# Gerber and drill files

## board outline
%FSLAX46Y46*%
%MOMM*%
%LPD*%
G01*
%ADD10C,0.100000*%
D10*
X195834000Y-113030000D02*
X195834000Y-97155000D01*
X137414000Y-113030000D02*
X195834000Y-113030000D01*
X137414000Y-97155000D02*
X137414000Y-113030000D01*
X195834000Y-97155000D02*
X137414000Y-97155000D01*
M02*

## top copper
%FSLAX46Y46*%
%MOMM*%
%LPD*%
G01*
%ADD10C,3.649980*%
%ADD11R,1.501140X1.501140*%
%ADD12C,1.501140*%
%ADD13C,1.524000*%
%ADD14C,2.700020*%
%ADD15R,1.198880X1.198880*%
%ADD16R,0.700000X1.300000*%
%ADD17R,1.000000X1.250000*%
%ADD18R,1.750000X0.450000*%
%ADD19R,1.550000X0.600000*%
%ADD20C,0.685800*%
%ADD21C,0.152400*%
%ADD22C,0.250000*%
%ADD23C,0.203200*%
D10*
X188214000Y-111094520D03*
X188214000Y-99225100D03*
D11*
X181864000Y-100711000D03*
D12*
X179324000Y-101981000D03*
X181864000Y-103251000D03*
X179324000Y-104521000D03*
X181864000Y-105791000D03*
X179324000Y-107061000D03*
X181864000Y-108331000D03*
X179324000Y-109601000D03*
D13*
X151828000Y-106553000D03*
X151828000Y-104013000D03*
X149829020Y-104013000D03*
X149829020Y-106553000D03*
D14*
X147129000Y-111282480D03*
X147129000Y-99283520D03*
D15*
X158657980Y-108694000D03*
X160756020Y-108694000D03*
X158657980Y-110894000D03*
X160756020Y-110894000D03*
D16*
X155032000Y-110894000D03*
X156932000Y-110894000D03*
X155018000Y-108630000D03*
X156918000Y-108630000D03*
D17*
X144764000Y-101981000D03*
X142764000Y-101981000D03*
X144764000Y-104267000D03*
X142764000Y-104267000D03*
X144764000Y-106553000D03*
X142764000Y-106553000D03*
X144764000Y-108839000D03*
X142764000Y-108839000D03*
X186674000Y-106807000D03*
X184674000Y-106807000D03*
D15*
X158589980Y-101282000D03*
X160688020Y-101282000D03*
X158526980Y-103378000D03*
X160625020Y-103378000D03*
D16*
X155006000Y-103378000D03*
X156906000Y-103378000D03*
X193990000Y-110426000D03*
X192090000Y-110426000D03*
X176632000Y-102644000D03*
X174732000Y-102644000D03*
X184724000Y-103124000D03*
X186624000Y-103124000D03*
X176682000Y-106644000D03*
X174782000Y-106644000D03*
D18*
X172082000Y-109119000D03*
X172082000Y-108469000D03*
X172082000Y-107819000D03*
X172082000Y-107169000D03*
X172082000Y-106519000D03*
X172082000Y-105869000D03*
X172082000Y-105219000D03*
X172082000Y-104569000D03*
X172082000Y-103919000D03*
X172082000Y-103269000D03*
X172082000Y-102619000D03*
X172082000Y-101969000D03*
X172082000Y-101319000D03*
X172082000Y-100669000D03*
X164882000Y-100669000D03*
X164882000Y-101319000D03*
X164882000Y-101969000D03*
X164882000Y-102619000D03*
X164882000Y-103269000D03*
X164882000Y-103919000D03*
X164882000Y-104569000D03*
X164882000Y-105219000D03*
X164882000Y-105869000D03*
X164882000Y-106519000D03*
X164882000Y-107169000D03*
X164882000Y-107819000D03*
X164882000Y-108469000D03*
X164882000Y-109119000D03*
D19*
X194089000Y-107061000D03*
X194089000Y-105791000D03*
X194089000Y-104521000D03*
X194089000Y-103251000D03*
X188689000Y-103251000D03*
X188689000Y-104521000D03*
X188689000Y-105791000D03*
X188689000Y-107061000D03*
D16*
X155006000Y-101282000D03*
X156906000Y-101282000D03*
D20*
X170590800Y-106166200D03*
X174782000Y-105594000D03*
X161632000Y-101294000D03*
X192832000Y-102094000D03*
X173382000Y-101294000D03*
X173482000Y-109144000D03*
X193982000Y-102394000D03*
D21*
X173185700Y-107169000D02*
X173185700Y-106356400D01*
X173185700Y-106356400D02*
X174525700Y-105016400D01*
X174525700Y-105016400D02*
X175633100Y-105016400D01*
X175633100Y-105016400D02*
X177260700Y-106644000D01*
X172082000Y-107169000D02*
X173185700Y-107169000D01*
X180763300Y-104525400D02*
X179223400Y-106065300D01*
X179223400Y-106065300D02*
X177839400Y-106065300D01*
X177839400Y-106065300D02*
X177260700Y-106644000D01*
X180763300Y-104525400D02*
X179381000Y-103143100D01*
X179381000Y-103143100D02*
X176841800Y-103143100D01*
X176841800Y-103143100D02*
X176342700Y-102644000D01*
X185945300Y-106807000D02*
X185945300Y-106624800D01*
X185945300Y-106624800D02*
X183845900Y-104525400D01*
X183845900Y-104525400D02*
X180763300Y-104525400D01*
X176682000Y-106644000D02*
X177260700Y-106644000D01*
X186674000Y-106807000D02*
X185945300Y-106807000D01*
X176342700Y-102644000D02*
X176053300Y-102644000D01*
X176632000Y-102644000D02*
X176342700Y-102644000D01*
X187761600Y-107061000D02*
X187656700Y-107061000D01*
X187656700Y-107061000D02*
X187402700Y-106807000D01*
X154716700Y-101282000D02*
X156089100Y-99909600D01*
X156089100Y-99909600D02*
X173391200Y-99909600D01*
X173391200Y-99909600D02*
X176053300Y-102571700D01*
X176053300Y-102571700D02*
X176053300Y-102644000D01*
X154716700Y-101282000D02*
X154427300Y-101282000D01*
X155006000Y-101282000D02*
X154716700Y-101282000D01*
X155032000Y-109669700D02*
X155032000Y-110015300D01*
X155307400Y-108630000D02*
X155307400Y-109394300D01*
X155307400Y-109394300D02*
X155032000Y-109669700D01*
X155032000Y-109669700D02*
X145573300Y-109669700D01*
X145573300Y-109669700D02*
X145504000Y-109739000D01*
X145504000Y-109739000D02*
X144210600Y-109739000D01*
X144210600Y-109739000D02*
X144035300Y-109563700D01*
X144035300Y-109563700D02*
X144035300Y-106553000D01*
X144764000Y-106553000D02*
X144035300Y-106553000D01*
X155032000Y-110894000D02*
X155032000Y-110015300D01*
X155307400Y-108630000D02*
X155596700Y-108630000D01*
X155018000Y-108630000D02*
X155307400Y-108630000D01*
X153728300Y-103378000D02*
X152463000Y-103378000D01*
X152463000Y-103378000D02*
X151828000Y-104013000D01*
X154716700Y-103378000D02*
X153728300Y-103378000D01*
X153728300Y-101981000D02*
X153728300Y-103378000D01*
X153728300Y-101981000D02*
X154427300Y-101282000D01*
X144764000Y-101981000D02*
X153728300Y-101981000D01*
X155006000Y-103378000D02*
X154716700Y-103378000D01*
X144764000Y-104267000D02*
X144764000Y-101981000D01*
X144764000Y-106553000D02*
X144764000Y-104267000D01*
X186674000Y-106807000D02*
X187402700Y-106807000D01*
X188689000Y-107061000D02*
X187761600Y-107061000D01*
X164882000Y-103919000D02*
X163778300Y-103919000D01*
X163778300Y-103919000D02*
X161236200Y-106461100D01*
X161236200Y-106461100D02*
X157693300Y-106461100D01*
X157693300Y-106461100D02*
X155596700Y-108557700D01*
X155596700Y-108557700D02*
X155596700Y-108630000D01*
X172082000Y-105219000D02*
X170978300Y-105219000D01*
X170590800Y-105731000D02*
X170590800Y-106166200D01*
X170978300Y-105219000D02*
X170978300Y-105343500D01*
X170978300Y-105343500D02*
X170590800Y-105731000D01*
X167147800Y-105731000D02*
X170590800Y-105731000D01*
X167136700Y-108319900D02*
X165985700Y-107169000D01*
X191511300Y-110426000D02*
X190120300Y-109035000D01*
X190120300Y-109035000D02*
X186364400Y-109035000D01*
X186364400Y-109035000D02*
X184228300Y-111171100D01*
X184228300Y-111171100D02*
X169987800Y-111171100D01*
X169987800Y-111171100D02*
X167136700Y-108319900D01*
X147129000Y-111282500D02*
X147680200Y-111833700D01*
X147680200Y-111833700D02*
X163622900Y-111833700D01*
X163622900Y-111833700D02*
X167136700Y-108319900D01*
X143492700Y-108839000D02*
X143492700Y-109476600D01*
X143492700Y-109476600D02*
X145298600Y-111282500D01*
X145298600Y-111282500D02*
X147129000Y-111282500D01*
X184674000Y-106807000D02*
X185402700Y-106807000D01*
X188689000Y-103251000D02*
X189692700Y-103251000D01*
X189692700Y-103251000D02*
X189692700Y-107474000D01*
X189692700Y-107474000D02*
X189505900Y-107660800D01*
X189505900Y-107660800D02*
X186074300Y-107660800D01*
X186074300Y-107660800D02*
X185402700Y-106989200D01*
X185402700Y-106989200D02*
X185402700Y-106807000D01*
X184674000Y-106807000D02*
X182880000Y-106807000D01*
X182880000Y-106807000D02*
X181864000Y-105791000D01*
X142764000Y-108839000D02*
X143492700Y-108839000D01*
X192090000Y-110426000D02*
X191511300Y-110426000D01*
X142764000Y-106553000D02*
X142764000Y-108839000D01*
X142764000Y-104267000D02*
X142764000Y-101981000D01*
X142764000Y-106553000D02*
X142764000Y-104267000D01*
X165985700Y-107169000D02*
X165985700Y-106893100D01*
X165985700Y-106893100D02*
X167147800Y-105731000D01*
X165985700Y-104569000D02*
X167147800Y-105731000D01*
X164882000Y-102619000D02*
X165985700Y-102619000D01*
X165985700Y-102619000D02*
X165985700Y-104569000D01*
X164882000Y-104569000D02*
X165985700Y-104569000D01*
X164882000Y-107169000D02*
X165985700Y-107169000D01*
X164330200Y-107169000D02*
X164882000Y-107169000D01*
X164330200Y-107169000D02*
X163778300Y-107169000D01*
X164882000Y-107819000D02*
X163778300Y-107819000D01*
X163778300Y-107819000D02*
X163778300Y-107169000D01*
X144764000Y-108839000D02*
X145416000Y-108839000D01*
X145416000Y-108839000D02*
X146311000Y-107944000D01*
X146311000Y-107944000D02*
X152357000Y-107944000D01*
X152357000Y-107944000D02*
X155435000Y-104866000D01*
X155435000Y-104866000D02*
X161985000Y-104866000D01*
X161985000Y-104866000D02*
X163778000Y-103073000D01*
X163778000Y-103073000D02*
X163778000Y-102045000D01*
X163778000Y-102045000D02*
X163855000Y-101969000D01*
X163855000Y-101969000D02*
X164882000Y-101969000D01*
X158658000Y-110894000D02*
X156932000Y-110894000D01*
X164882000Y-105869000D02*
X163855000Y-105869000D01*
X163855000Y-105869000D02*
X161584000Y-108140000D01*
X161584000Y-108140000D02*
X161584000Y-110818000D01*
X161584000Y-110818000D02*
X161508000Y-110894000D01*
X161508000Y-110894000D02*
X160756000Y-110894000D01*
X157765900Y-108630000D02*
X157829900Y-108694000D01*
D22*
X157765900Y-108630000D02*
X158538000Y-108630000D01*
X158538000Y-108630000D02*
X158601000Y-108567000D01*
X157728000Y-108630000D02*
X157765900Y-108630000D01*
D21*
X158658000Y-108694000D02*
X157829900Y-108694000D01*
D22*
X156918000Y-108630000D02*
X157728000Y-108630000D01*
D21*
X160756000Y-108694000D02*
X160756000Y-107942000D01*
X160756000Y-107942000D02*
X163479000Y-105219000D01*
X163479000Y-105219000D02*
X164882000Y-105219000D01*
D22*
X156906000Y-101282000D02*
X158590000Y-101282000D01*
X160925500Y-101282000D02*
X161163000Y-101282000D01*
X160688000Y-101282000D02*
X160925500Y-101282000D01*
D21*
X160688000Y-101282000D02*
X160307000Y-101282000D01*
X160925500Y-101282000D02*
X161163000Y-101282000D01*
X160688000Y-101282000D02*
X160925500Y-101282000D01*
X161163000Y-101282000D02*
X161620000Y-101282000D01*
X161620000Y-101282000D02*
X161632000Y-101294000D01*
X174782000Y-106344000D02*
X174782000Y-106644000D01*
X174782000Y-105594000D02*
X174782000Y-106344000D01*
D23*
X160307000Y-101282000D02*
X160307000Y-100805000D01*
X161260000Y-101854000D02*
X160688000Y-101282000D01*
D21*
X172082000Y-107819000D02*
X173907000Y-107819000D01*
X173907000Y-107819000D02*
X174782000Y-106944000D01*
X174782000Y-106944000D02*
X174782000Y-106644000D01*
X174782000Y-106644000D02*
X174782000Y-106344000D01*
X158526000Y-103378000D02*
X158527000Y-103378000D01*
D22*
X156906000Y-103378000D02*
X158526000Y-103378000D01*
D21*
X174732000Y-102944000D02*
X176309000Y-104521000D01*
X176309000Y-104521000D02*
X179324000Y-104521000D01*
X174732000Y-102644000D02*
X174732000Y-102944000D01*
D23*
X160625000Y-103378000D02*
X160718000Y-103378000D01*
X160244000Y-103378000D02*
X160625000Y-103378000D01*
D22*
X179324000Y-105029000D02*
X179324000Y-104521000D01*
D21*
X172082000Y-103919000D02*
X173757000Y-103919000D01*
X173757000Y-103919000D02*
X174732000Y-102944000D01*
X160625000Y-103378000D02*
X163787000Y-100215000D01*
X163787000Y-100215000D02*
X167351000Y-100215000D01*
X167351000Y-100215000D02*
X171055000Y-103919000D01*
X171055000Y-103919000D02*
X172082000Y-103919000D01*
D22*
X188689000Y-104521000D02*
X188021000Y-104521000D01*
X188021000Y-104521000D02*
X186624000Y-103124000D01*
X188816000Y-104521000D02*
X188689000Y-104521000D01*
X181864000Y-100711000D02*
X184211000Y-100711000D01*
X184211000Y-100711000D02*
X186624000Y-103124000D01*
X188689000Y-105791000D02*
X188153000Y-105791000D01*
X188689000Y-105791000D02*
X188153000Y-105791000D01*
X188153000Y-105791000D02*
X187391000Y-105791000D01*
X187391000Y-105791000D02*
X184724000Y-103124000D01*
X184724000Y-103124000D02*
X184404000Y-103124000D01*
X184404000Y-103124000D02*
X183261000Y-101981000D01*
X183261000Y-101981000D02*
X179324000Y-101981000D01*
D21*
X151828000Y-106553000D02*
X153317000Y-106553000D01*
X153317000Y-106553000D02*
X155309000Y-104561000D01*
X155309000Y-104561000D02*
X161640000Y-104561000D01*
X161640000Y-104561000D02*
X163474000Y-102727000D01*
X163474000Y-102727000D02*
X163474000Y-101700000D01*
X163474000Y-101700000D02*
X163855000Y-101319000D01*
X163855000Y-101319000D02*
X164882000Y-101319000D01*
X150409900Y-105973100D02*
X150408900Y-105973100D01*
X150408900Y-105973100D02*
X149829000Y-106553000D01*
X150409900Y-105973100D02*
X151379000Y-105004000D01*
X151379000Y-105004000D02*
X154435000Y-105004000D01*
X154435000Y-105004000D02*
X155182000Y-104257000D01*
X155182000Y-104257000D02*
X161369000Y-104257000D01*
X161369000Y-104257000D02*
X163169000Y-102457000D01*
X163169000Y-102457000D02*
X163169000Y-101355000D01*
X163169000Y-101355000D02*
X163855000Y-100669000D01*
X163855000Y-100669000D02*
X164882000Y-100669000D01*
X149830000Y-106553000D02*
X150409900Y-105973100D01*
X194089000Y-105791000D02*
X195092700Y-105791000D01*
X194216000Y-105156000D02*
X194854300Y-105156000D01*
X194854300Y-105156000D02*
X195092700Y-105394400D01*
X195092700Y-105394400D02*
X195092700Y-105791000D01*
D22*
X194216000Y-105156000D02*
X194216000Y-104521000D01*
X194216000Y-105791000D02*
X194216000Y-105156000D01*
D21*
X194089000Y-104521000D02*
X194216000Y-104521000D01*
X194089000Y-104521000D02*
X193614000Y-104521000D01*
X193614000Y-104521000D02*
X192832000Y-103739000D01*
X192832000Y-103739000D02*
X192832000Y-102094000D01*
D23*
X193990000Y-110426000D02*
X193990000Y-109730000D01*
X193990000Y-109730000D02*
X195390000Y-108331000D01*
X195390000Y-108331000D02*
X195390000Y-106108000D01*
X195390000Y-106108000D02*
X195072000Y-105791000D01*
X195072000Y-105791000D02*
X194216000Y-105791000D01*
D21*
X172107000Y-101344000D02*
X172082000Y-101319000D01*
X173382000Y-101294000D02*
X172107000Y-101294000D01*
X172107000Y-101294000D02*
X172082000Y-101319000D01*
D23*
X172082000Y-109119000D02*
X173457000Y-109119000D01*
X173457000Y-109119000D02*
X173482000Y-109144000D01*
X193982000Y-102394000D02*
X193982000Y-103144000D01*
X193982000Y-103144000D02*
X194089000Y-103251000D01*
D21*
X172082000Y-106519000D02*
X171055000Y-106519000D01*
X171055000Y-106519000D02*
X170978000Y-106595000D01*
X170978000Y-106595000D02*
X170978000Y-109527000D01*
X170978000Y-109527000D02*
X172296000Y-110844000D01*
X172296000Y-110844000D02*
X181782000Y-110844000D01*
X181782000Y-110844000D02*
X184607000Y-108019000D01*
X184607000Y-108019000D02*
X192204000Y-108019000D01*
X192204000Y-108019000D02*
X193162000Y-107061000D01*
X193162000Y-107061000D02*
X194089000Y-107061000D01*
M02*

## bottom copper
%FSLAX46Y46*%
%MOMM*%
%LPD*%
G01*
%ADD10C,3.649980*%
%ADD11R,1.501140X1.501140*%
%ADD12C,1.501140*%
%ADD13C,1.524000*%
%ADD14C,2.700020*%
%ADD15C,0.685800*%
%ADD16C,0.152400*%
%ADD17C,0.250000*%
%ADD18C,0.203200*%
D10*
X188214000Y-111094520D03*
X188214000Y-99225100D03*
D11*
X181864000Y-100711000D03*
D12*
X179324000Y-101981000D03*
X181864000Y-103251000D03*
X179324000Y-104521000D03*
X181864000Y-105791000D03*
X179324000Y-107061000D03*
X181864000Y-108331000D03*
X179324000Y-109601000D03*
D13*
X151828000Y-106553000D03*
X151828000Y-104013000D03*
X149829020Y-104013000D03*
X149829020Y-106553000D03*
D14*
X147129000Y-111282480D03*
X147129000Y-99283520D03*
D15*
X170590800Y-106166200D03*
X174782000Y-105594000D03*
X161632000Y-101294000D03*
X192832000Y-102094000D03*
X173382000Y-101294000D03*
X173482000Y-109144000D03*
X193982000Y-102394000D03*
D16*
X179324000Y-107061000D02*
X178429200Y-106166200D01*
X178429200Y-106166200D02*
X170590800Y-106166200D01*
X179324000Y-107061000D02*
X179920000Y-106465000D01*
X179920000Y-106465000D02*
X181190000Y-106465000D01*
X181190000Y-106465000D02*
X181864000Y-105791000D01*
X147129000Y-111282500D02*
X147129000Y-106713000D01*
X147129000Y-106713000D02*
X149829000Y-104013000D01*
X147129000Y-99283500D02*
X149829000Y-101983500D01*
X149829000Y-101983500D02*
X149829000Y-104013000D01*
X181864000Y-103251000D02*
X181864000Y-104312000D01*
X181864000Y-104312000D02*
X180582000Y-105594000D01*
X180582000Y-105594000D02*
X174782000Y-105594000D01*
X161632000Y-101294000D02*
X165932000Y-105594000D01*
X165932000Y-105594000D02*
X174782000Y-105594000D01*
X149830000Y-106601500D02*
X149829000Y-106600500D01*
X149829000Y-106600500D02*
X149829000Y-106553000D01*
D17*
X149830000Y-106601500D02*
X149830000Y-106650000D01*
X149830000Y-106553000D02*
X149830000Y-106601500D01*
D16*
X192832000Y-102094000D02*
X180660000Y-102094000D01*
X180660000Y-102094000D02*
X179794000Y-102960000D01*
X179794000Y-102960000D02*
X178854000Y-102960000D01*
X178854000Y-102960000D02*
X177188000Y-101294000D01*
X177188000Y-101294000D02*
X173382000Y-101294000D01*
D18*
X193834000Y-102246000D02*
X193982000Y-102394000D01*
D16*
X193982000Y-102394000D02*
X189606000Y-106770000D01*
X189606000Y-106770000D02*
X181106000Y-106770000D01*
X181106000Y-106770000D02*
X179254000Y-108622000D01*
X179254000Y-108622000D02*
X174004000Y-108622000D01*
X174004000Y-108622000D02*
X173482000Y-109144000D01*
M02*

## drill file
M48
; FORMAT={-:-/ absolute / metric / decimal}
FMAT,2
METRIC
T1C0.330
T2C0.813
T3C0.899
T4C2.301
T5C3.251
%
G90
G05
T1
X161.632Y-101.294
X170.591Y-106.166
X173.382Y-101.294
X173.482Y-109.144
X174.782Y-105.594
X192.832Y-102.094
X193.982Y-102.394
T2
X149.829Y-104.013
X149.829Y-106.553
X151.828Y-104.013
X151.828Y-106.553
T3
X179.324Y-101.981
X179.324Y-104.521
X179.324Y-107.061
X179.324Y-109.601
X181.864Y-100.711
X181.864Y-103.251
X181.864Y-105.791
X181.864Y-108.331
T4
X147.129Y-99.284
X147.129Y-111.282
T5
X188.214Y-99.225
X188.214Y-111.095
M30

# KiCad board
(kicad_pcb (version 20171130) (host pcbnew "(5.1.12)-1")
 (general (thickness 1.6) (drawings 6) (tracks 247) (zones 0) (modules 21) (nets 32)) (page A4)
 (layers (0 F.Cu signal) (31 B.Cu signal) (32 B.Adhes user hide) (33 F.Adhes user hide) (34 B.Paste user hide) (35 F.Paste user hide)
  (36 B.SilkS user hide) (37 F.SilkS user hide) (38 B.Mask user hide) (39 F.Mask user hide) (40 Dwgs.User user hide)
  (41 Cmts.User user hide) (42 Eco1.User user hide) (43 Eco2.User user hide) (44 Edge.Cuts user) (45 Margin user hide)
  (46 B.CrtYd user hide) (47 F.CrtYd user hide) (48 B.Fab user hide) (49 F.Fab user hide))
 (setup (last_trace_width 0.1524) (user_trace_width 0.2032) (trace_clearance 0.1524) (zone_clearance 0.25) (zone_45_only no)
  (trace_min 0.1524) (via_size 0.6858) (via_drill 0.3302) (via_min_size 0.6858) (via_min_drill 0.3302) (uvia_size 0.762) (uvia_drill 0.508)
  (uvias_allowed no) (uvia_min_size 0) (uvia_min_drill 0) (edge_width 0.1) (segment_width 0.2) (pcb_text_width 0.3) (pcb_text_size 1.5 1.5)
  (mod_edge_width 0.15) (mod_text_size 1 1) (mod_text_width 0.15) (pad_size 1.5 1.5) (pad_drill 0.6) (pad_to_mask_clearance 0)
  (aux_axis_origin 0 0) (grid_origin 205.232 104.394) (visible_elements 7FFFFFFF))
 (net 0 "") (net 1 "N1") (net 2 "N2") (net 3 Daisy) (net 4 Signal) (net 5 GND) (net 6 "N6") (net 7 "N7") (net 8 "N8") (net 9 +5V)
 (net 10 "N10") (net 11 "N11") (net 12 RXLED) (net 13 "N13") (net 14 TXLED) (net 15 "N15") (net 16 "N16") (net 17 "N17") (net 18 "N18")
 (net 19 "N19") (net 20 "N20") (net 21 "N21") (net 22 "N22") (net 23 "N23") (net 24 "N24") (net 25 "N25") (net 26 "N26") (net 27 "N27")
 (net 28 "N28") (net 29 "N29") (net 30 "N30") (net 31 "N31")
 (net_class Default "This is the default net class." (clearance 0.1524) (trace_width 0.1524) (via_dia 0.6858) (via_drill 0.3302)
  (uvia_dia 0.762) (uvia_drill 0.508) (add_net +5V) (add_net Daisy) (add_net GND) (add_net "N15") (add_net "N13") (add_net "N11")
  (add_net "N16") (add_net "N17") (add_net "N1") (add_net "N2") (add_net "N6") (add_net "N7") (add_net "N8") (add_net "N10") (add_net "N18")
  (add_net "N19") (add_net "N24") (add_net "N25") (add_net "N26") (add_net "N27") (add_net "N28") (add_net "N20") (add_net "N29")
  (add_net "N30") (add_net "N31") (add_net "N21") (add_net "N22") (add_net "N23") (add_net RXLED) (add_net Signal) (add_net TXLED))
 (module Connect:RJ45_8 (layer B.Cu) (at 188.214 105.156 270)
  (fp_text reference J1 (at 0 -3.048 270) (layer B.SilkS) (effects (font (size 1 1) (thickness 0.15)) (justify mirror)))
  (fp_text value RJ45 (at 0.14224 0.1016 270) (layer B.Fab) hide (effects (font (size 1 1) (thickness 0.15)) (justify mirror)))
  (pad Hole np_thru_hole circle (at 5.93852 0 270) (size 3.64998 3.64998) (drill 3.2512) (layers *.Cu *.SilkS *.Mask))
  (pad Hole np_thru_hole circle (at -5.9309 0 270) (size 3.64998 3.64998) (drill 3.2512) (layers *.Cu *.SilkS *.Mask))
  (pad 1 thru_hole rect (at -4.445 6.35 270) (size 1.50114 1.50114) (drill 0.89916) (layers *.Cu *.Mask B.SilkS) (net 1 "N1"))
  (pad 2 thru_hole circle (at -3.175 8.89 270) (size 1.50114 1.50114) (drill 0.89916) (layers *.Cu *.Mask B.SilkS) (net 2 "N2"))
  (pad 3 thru_hole circle (at -1.905 6.35 270) (size 1.50114 1.50114) (drill 0.89916) (layers *.Cu *.Mask B.SilkS) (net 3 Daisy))
  (pad 4 thru_hole circle (at -0.635 8.89 270) (size 1.50114 1.50114) (drill 0.89916) (layers *.Cu *.Mask B.SilkS) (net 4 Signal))
  (pad 5 thru_hole circle (at 0.635 6.35 270) (size 1.50114 1.50114) (drill 0.89916) (layers *.Cu *.Mask B.SilkS) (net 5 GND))
  (pad 6 thru_hole circle (at 1.905 8.89 270) (size 1.50114 1.50114) (drill 0.89916) (layers *.Cu *.Mask B.SilkS) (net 5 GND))
  (pad 7 thru_hole circle (at 3.175 6.35 270) (size 1.50114 1.50114) (drill 0.89916) (layers *.Cu *.Mask B.SilkS) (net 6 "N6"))
  (pad 8 thru_hole circle (at 4.445 8.89 270) (size 1.50114 1.50114) (drill 0.89916) (layers *.Cu *.Mask B.SilkS) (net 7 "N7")))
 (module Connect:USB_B (layer B.Cu) (at 151.828 104.013 180)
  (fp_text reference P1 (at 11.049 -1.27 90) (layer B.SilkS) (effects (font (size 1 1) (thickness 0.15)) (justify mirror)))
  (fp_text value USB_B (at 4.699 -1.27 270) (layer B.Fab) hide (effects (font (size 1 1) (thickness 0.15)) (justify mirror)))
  (pad 2 thru_hole circle (at 0 -2.54 270) (size 1.524 1.524) (drill 0.8128) (layers *.Cu *.Mask B.SilkS) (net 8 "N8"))
  (pad 1 thru_hole circle (at 0 0 270) (size 1.524 1.524) (drill 0.8128) (layers *.Cu *.Mask B.SilkS) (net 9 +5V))
  (pad 4 thru_hole circle (at 1.99898 0 270) (size 1.524 1.524) (drill 0.8128) (layers *.Cu *.Mask B.SilkS) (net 5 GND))
  (pad 3 thru_hole circle (at 1.99898 -2.54 270) (size 1.524 1.524) (drill 0.8128) (layers *.Cu *.Mask B.SilkS) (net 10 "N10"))
  (pad 5 thru_hole circle (at 4.699 -7.26948 270) (size 2.70002 2.70002) (drill 2.30124) (layers *.Cu *.Mask B.SilkS) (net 5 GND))
  (pad 5 thru_hole circle (at 4.699 4.72948 270) (size 2.70002 2.70002) (drill 2.30124) (layers *.Cu *.Mask B.SilkS) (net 5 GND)))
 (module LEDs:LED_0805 (layer F.Cu) (at 159.707 108.694 180)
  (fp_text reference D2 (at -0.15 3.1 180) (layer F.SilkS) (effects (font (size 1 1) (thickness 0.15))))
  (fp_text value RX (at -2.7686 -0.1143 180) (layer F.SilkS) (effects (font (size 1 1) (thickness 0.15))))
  (pad 2 smd rect (at 1.04902 0) (size 1.19888 1.19888) (layers F.Cu F.Paste F.Mask) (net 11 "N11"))
  (pad 1 smd rect (at -1.04902 0) (size 1.19888 1.19888) (layers F.Cu F.Paste F.Mask) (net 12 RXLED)))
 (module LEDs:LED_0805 (layer F.Cu) (at 159.707 110.894 180)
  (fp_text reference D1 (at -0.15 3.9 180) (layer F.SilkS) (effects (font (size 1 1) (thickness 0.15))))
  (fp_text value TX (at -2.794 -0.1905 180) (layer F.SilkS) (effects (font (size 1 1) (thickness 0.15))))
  (pad 2 smd rect (at 1.04902 0) (size 1.19888 1.19888) (layers F.Cu F.Paste F.Mask) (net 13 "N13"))
  (pad 1 smd rect (at -1.04902 0) (size 1.19888 1.19888) (layers F.Cu F.Paste F.Mask) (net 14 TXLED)))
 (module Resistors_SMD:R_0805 (layer F.Cu) (at 155.982 110.894)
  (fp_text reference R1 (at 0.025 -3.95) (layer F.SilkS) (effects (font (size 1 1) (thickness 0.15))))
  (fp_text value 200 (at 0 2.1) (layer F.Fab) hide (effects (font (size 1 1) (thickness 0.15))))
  (pad 1 smd rect (at -0.95 0) (size 0.7 1.3) (layers F.Cu F.Paste F.Mask) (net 9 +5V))
  (pad 2 smd rect (at 0.95 0) (size 0.7 1.3) (layers F.Cu F.Paste F.Mask) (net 13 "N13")))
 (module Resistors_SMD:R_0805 (layer F.Cu) (at 155.968 108.63)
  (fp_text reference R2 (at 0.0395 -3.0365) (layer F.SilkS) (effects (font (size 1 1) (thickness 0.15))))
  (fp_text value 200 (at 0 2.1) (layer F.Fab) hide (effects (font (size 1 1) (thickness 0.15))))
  (pad 1 smd rect (at -0.95 0) (size 0.7 1.3) (layers F.Cu F.Paste F.Mask) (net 9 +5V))
  (pad 2 smd rect (at 0.95 0) (size 0.7 1.3) (layers F.Cu F.Paste F.Mask) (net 11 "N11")))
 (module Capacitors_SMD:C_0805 (layer F.Cu) (at 143.764 101.981 180)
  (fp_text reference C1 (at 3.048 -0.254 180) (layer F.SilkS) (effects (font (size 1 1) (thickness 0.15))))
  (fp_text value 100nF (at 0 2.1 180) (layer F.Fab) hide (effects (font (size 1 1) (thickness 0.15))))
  (pad 1 smd rect (at -1 0 180) (size 1 1.25) (layers F.Cu F.Paste F.Mask) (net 9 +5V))
  (pad 2 smd rect (at 1 0 180) (size 1 1.25) (layers F.Cu F.Paste F.Mask) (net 5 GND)))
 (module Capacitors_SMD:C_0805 (layer F.Cu) (at 143.764 104.267 180)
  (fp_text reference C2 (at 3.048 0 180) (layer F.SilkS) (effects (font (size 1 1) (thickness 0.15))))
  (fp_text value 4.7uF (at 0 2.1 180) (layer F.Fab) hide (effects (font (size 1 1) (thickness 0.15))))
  (pad 1 smd rect (at -1 0 180) (size 1 1.25) (layers F.Cu F.Paste F.Mask) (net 9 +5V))
  (pad 2 smd rect (at 1 0 180) (size 1 1.25) (layers F.Cu F.Paste F.Mask) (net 5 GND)))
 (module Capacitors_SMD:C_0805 (layer F.Cu) (at 143.764 106.553 180)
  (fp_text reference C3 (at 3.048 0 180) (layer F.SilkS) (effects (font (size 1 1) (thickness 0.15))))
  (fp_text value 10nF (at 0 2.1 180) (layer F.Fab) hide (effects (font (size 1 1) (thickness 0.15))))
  (pad 1 smd rect (at -1 0 180) (size 1 1.25) (layers F.Cu F.Paste F.Mask) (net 9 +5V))
  (pad 2 smd rect (at 1 0 180) (size 1 1.25) (layers F.Cu F.Paste F.Mask) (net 5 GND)))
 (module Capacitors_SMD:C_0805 (layer F.Cu) (at 143.764 108.839 180)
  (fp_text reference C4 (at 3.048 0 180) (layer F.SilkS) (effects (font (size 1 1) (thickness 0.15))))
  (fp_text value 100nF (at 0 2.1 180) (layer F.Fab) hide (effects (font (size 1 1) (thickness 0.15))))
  (pad 1 smd rect (at -1 0 180) (size 1 1.25) (layers F.Cu F.Paste F.Mask) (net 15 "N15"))
  (pad 2 smd rect (at 1 0 180) (size 1 1.25) (layers F.Cu F.Paste F.Mask) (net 5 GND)))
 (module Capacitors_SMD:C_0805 (layer F.Cu) (at 185.674 106.807 180)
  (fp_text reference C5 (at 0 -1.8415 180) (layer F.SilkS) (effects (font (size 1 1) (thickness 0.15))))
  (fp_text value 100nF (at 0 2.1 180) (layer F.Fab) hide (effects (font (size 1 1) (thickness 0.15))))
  (pad 1 smd rect (at -1 0 180) (size 1 1.25) (layers F.Cu F.Paste F.Mask) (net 9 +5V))
  (pad 2 smd rect (at 1 0 180) (size 1 1.25) (layers F.Cu F.Paste F.Mask) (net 5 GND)))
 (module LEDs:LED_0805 (layer F.Cu) (at 159.639 101.282 180)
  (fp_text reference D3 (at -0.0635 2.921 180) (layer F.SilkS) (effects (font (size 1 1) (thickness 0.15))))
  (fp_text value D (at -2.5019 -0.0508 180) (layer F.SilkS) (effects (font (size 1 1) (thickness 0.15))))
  (pad 2 smd rect (at 1.04902 0) (size 1.19888 1.19888) (layers F.Cu F.Paste F.Mask) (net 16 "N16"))
  (pad 1 smd rect (at -1.04902 0) (size 1.19888 1.19888) (layers F.Cu F.Paste F.Mask) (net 3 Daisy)))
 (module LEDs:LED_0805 (layer F.Cu) (at 159.576 103.378 180)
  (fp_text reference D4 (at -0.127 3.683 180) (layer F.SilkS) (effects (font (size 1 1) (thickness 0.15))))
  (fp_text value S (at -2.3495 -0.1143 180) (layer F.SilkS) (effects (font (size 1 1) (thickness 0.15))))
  (pad 2 smd rect (at 1.04902 0) (size 1.19888 1.19888) (layers F.Cu F.Paste F.Mask) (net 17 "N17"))
  (pad 1 smd rect (at -1.04902 0) (size 1.19888 1.19888) (layers F.Cu F.Paste F.Mask) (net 4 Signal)))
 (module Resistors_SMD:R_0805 (layer F.Cu) (at 155.956 103.378)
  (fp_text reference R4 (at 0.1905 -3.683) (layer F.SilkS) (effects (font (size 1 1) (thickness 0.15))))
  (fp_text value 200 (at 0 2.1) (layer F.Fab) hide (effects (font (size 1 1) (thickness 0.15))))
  (pad 1 smd rect (at -0.95 0) (size 0.7 1.3) (layers F.Cu F.Paste F.Mask) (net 9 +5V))
  (pad 2 smd rect (at 0.95 0) (size 0.7 1.3) (layers F.Cu F.Paste F.Mask) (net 17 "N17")))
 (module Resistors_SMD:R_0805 (layer F.Cu) (at 193.04 110.426 180)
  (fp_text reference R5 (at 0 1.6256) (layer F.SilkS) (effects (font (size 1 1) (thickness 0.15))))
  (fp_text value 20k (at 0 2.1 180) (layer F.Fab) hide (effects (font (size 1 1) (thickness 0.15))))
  (pad 1 smd rect (at -0.95 0 180) (size 0.7 1.3) (layers F.Cu F.Paste F.Mask) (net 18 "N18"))
  (pad 2 smd rect (at 0.95 0 180) (size 0.7 1.3) (layers F.Cu F.Paste F.Mask) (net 5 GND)))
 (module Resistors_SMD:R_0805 (layer F.Cu) (at 175.682 102.644 180)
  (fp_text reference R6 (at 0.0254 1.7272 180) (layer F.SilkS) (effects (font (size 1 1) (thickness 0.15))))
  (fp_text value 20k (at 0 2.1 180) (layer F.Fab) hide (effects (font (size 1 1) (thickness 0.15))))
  (pad 1 smd rect (at -0.95 0 180) (size 0.7 1.3) (layers F.Cu F.Paste F.Mask) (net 9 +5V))
  (pad 2 smd rect (at 0.95 0 180) (size 0.7 1.3) (layers F.Cu F.Paste F.Mask) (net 4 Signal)))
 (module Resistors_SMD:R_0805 (layer F.Cu) (at 185.674 103.124)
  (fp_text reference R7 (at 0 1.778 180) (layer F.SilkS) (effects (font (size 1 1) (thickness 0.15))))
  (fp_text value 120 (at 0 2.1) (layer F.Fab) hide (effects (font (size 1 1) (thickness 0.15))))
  (pad 1 smd rect (at -0.95 0) (size 0.7 1.3) (layers F.Cu F.Paste F.Mask) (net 2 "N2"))
  (pad 2 smd rect (at 0.95 0) (size 0.7 1.3) (layers F.Cu F.Paste F.Mask) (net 1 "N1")))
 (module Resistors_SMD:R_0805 (layer F.Cu) (at 175.732 106.644 180)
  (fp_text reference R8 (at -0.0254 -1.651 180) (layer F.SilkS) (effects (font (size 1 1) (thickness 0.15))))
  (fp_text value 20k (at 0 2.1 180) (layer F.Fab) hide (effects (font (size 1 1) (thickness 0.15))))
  (pad 1 smd rect (at -0.95 0 180) (size 0.7 1.3) (layers F.Cu F.Paste F.Mask) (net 9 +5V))
  (pad 2 smd rect (at 0.95 0 180) (size 0.7 1.3) (layers F.Cu F.Paste F.Mask) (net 3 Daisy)))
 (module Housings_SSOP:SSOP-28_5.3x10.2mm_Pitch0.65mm (layer F.Cu) (at 168.482 104.894 180)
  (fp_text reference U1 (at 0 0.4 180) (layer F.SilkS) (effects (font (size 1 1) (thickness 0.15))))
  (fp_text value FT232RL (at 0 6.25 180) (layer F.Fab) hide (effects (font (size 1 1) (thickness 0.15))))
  (pad 1 smd rect (at -3.6 -4.225 180) (size 1.75 0.45) (layers F.Cu F.Paste F.Mask) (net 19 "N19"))
  (pad 2 smd rect (at -3.6 -3.575 180) (size 1.75 0.45) (layers F.Cu F.Paste F.Mask) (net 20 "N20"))
  (pad 3 smd rect (at -3.6 -2.925 180) (size 1.75 0.45) (layers F.Cu F.Paste F.Mask) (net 3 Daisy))
  (pad 4 smd rect (at -3.6 -2.275 180) (size 1.75 0.45) (layers F.Cu F.Paste F.Mask) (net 9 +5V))
  (pad 5 smd rect (at -3.6 -1.625 180) (size 1.75 0.45) (layers F.Cu F.Paste F.Mask) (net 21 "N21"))
  (pad 6 smd rect (at -3.6 -0.975 180) (size 1.75 0.45) (layers F.Cu F.Paste F.Mask) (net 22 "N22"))
  (pad 7 smd rect (at -3.6 -0.325 180) (size 1.75 0.45) (layers F.Cu F.Paste F.Mask) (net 5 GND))
  (pad 8 smd rect (at -3.6 0.325 180) (size 1.75 0.45) (layers F.Cu F.Paste F.Mask) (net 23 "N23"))
  (pad 9 smd rect (at -3.6 0.975 180) (size 1.75 0.45) (layers F.Cu F.Paste F.Mask) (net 4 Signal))
  (pad 10 smd rect (at -3.6 1.625 180) (size 1.75 0.45) (layers F.Cu F.Paste F.Mask) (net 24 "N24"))
  (pad 11 smd rect (at -3.6 2.275 180) (size 1.75 0.45) (layers F.Cu F.Paste F.Mask) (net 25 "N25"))
  (pad 12 smd rect (at -3.6 2.925 180) (size 1.75 0.45) (layers F.Cu F.Paste F.Mask) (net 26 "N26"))
  (pad 13 smd rect (at -3.6 3.575 180) (size 1.75 0.45) (layers F.Cu F.Paste F.Mask) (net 18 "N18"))
  (pad 14 smd rect (at -3.6 4.225 180) (size 1.75 0.45) (layers F.Cu F.Paste F.Mask) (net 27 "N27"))
  (pad 15 smd rect (at 3.6 4.225 180) (size 1.75 0.45) (layers F.Cu F.Paste F.Mask) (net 10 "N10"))
  (pad 16 smd rect (at 3.6 3.575 180) (size 1.75 0.45) (layers F.Cu F.Paste F.Mask) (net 8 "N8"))
  (pad 17 smd rect (at 3.6 2.925 180) (size 1.75 0.45) (layers F.Cu F.Paste F.Mask) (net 15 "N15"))
  (pad 18 smd rect (at 3.6 2.275 180) (size 1.75 0.45) (layers F.Cu F.Paste F.Mask) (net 5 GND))
  (pad 19 smd rect (at 3.6 1.625 180) (size 1.75 0.45) (layers F.Cu F.Paste F.Mask) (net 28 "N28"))
  (pad 20 smd rect (at 3.6 0.975 180) (size 1.75 0.45) (layers F.Cu F.Paste F.Mask) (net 9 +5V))
  (pad 21 smd rect (at 3.6 0.325 180) (size 1.75 0.45) (layers F.Cu F.Paste F.Mask) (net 5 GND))
  (pad 22 smd rect (at 3.6 -0.325 180) (size 1.75 0.45) (layers F.Cu F.Paste F.Mask) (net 12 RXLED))
  (pad 23 smd rect (at 3.6 -0.975 180) (size 1.75 0.45) (layers F.Cu F.Paste F.Mask) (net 14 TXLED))
  (pad 24 smd rect (at 3.6 -1.625 180) (size 1.75 0.45) (layers F.Cu F.Paste F.Mask) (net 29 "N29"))
  (pad 25 smd rect (at 3.6 -2.275 180) (size 1.75 0.45) (layers F.Cu F.Paste F.Mask) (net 5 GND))
  (pad 26 smd rect (at 3.6 -2.925 180) (size 1.75 0.45) (layers F.Cu F.Paste F.Mask) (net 5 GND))
  (pad 27 smd rect (at 3.6 -3.575 180) (size 1.75 0.45) (layers F.Cu F.Paste F.Mask) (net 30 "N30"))
  (pad 28 smd rect (at 3.6 -4.225 180) (size 1.75 0.45) (layers F.Cu F.Paste F.Mask) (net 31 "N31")))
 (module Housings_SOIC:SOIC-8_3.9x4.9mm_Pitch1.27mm (layer F.Cu) (at 191.389 105.156 180)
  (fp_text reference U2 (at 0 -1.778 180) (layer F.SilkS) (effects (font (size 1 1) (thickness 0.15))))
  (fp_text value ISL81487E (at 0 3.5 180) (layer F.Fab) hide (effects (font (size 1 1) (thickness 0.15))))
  (pad 1 smd rect (at -2.7 -1.905 180) (size 1.55 0.6) (layers F.Cu F.Paste F.Mask) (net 21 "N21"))
  (pad 2 smd rect (at -2.7 -0.635 180) (size 1.55 0.6) (layers F.Cu F.Paste F.Mask) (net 18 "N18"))
  (pad 3 smd rect (at -2.7 0.635 180) (size 1.55 0.6) (layers F.Cu F.Paste F.Mask) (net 18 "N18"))
  (pad 4 smd rect (at -2.7 1.905 180) (size 1.55 0.6) (layers F.Cu F.Paste F.Mask) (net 19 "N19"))
  (pad 5 smd rect (at 2.7 1.905 180) (size 1.55 0.6) (layers F.Cu F.Paste F.Mask) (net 5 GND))
  (pad 6 smd rect (at 2.7 0.635 180) (size 1.55 0.6) (layers F.Cu F.Paste F.Mask) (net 1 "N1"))
  (pad 7 smd rect (at 2.7 -0.635 180) (size 1.55 0.6) (layers F.Cu F.Paste F.Mask) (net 2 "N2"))
  (pad 8 smd rect (at 2.7 -1.905 180) (size 1.55 0.6) (layers F.Cu F.Paste F.Mask) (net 9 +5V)))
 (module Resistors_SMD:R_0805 (layer F.Cu) (at 155.956 101.282)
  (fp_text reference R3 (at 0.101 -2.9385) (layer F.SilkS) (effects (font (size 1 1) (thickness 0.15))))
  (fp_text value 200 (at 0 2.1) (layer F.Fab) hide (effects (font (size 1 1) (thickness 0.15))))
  (pad 1 smd rect (at -0.95 0) (size 0.7 1.3) (layers F.Cu F.Paste F.Mask) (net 9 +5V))
  (pad 2 smd rect (at 0.95 0) (size 0.7 1.3) (layers F.Cu F.Paste F.Mask) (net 16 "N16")))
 (gr_line (start 195.834 113.03) (end 195.834 97.155) (angle 90) (layer Edge.Cuts) (width 0.1))
 (gr_line (start 137.414 113.03) (end 195.834 113.03) (angle 90) (layer Edge.Cuts) (width 0.1))
 (gr_line (start 137.414 97.155) (end 137.414 113.03) (angle 90) (layer Edge.Cuts) (width 0.1))
 (gr_line (start 195.834 97.155) (end 137.414 97.155) (angle 90) (layer Edge.Cuts) (width 0.1))
 (segment (start 173.1857 107.169) (end 173.1857 106.3564) (width 0.1524) (layer F.Cu) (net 9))
 (segment (start 173.1857 106.3564) (end 174.5257 105.0164) (width 0.1524) (layer F.Cu) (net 9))
 (segment (start 174.5257 105.0164) (end 175.6331 105.0164) (width 0.1524) (layer F.Cu) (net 9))
 (segment (start 175.6331 105.0164) (end 177.2607 106.644) (width 0.1524) (layer F.Cu) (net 9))
 (segment (start 172.082 107.169) (end 173.1857 107.169) (width 0.1524) (layer F.Cu) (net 9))
 (segment (start 180.7633 104.5254) (end 179.2234 106.0653) (width 0.1524) (layer F.Cu) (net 9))
 (segment (start 179.2234 106.0653) (end 177.8394 106.0653) (width 0.1524) (layer F.Cu) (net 9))
 (segment (start 177.8394 106.0653) (end 177.2607 106.644) (width 0.1524) (layer F.Cu) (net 9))
 (segment (start 180.7633 104.5254) (end 179.381 103.1431) (width 0.1524) (layer F.Cu) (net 9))
 (segment (start 179.381 103.1431) (end 176.8418 103.1431) (width 0.1524) (layer F.Cu) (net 9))
 (segment (start 176.8418 103.1431) (end 176.3427 102.644) (width 0.1524) (layer F.Cu) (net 9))
 (segment (start 185.9453 106.807) (end 185.9453 106.6248) (width 0.1524) (layer F.Cu) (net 9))
 (segment (start 185.9453 106.6248) (end 183.8459 104.5254) (width 0.1524) (layer F.Cu) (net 9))
 (segment (start 183.8459 104.5254) (end 180.7633 104.5254) (width 0.1524) (layer F.Cu) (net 9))
 (segment (start 176.682 106.644) (end 177.2607 106.644) (width 0.1524) (layer F.Cu) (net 9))
 (segment (start 186.674 106.807) (end 185.9453 106.807) (width 0.1524) (layer F.Cu) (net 9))
 (segment (start 176.3427 102.644) (end 176.0533 102.644) (width 0.1524) (layer F.Cu) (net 9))
 (segment (start 176.632 102.644) (end 176.3427 102.644) (width 0.1524) (layer F.Cu) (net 9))
 (segment (start 187.7616 107.061) (end 187.6567 107.061) (width 0.1524) (layer F.Cu) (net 9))
 (segment (start 187.6567 107.061) (end 187.4027 106.807) (width 0.1524) (layer F.Cu) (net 9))
 (segment (start 154.7167 101.282) (end 156.0891 99.9096) (width 0.1524) (layer F.Cu) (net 9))
 (segment (start 156.0891 99.9096) (end 173.3912 99.9096) (width 0.1524) (layer F.Cu) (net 9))
 (segment (start 173.3912 99.9096) (end 176.0533 102.5717) (width 0.1524) (layer F.Cu) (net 9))
 (segment (start 176.0533 102.5717) (end 176.0533 102.644) (width 0.1524) (layer F.Cu) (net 9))
 (segment (start 154.7167 101.282) (end 154.4273 101.282) (width 0.1524) (layer F.Cu) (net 9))
 (segment (start 155.006 101.282) (end 154.7167 101.282) (width 0.1524) (layer F.Cu) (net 9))
 (segment (start 155.032 109.6697) (end 155.032 110.0153) (width 0.1524) (layer F.Cu) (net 9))
 (segment (start 155.3074 108.63) (end 155.3074 109.3943) (width 0.1524) (layer F.Cu) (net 9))
 (segment (start 155.3074 109.3943) (end 155.032 109.6697) (width 0.1524) (layer F.Cu) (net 9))
 (segment (start 155.032 109.6697) (end 145.5733 109.6697) (width 0.1524) (layer F.Cu) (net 9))
 (segment (start 145.5733 109.6697) (end 145.504 109.739) (width 0.1524) (layer F.Cu) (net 9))
 (segment (start 145.504 109.739) (end 144.2106 109.739) (width 0.1524) (layer F.Cu) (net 9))
 (segment (start 144.2106 109.739) (end 144.0353 109.5637) (width 0.1524) (layer F.Cu) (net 9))
 (segment (start 144.0353 109.5637) (end 144.0353 106.553) (width 0.1524) (layer F.Cu) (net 9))
 (segment (start 144.764 106.553) (end 144.0353 106.553) (width 0.1524) (layer F.Cu) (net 9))
 (segment (start 155.032 110.894) (end 155.032 110.0153) (width 0.1524) (layer F.Cu) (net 9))
 (segment (start 155.3074 108.63) (end 155.5967 108.63) (width 0.1524) (layer F.Cu) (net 9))
 (segment (start 155.018 108.63) (end 155.3074 108.63) (width 0.1524) (layer F.Cu) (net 9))
 (segment (start 153.7283 103.378) (end 152.463 103.378) (width 0.1524) (layer F.Cu) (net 9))
 (segment (start 152.463 103.378) (end 151.828 104.013) (width 0.1524) (layer F.Cu) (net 9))
 (segment (start 154.7167 103.378) (end 153.7283 103.378) (width 0.1524) (layer F.Cu) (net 9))
 (segment (start 153.7283 101.981) (end 153.7283 103.378) (width 0.1524) (layer F.Cu) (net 9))
 (segment (start 153.7283 101.981) (end 154.4273 101.282) (width 0.1524) (layer F.Cu) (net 9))
 (segment (start 144.764 101.981) (end 153.7283 101.981) (width 0.1524) (layer F.Cu) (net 9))
 (segment (start 155.006 103.378) (end 154.7167 103.378) (width 0.1524) (layer F.Cu) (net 9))
 (segment (start 144.764 104.267) (end 144.764 101.981) (width 0.1524) (layer F.Cu) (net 9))
 (segment (start 144.764 106.553) (end 144.764 104.267) (width 0.1524) (layer F.Cu) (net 9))
 (segment (start 186.674 106.807) (end 187.4027 106.807) (width 0.1524) (layer F.Cu) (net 9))
 (segment (start 188.689 107.061) (end 187.7616 107.061) (width 0.1524) (layer F.Cu) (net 9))
 (segment (start 164.882 103.919) (end 163.7783 103.919) (width 0.1524) (layer F.Cu) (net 9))
 (segment (start 163.7783 103.919) (end 161.2362 106.4611) (width 0.1524) (layer F.Cu) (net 9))
 (segment (start 161.2362 106.4611) (end 157.6933 106.4611) (width 0.1524) (layer F.Cu) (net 9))
 (segment (start 157.6933 106.4611) (end 155.5967 108.5577) (width 0.1524) (layer F.Cu) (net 9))
 (segment (start 155.5967 108.5577) (end 155.5967 108.63) (width 0.1524) (layer F.Cu) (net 9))
 (segment (start 172.082 105.219) (end 170.9783 105.219) (width 0.1524) (layer F.Cu) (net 5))
 (segment (start 170.5908 105.731) (end 170.5908 106.1662) (width 0.1524) (layer F.Cu) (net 5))
 (segment (start 170.9783 105.219) (end 170.9783 105.3435) (width 0.1524) (layer F.Cu) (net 5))
 (segment (start 170.9783 105.3435) (end 170.5908 105.731) (width 0.1524) (layer F.Cu) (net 5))
 (segment (start 167.1478 105.731) (end 170.5908 105.731) (width 0.1524) (layer F.Cu) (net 5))
 (segment (start 179.324 107.061) (end 178.4292 106.1662) (width 0.1524) (layer B.Cu) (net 5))
 (segment (start 178.4292 106.1662) (end 170.5908 106.1662) (width 0.1524) (layer B.Cu) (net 5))
 (segment (start 179.324 107.061) (end 179.92 106.465) (width 0.1524) (layer B.Cu) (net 5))
 (segment (start 179.92 106.465) (end 181.19 106.465) (width 0.1524) (layer B.Cu) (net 5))
 (segment (start 181.19 106.465) (end 181.864 105.791) (width 0.1524) (layer B.Cu) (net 5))
 (segment (start 167.1367 108.3199) (end 165.9857 107.169) (width 0.1524) (layer F.Cu) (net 5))
 (segment (start 191.5113 110.426) (end 190.1203 109.035) (width 0.1524) (layer F.Cu) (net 5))
 (segment (start 190.1203 109.035) (end 186.3644 109.035) (width 0.1524) (layer F.Cu) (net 5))
 (segment (start 186.3644 109.035) (end 184.2283 111.1711) (width 0.1524) (layer F.Cu) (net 5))
 (segment (start 184.2283 111.1711) (end 169.9878 111.1711) (width 0.1524) (layer F.Cu) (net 5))
 (segment (start 169.9878 111.1711) (end 167.1367 108.3199) (width 0.1524) (layer F.Cu) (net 5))
 (segment (start 147.129 111.2825) (end 147.6802 111.8337) (width 0.1524) (layer F.Cu) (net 5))
 (segment (start 147.6802 111.8337) (end 163.6229 111.8337) (width 0.1524) (layer F.Cu) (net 5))
 (segment (start 163.6229 111.8337) (end 167.1367 108.3199) (width 0.1524) (layer F.Cu) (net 5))
 (segment (start 143.4927 108.839) (end 143.4927 109.4766) (width 0.1524) (layer F.Cu) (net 5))
 (segment (start 143.4927 109.4766) (end 145.2986 111.2825) (width 0.1524) (layer F.Cu) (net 5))
 (segment (start 145.2986 111.2825) (end 147.129 111.2825) (width 0.1524) (layer F.Cu) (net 5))
 (segment (start 184.674 106.807) (end 185.4027 106.807) (width 0.1524) (layer F.Cu) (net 5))
 (segment (start 188.689 103.251) (end 189.6927 103.251) (width 0.1524) (layer F.Cu) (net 5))
 (segment (start 189.6927 103.251) (end 189.6927 107.474) (width 0.1524) (layer F.Cu) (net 5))
 (segment (start 189.6927 107.474) (end 189.5059 107.6608) (width 0.1524) (layer F.Cu) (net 5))
 (segment (start 189.5059 107.6608) (end 186.0743 107.6608) (width 0.1524) (layer F.Cu) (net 5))
 (segment (start 186.0743 107.6608) (end 185.4027 106.9892) (width 0.1524) (layer F.Cu) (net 5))
 (segment (start 185.4027 106.9892) (end 185.4027 106.807) (width 0.1524) (layer F.Cu) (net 5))
 (segment (start 184.674 106.807) (end 182.88 106.807) (width 0.1524) (layer F.Cu) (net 5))
 (segment (start 182.88 106.807) (end 181.864 105.791) (width 0.1524) (layer F.Cu) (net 5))
 (segment (start 142.764 108.839) (end 143.4927 108.839) (width 0.1524) (layer F.Cu) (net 5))
 (segment (start 147.129 111.2825) (end 147.129 106.713) (width 0.1524) (layer B.Cu) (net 5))
 (segment (start 147.129 106.713) (end 149.829 104.013) (width 0.1524) (layer B.Cu) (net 5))
 (segment (start 147.129 99.2835) (end 149.829 101.9835) (width 0.1524) (layer B.Cu) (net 5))
 (segment (start 149.829 101.9835) (end 149.829 104.013) (width 0.1524) (layer B.Cu) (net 5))
 (segment (start 192.09 110.426) (end 191.5113 110.426) (width 0.1524) (layer F.Cu) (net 5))
 (segment (start 142.764 106.553) (end 142.764 108.839) (width 0.1524) (layer F.Cu) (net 5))
 (segment (start 142.764 104.267) (end 142.764 101.981) (width 0.1524) (layer F.Cu) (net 5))
 (segment (start 142.764 106.553) (end 142.764 104.267) (width 0.1524) (layer F.Cu) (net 5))
 (segment (start 165.9857 107.169) (end 165.9857 106.8931) (width 0.1524) (layer F.Cu) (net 5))
 (segment (start 165.9857 106.8931) (end 167.1478 105.731) (width 0.1524) (layer F.Cu) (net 5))
 (segment (start 165.9857 104.569) (end 167.1478 105.731) (width 0.1524) (layer F.Cu) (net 5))
 (segment (start 164.882 102.619) (end 165.9857 102.619) (width 0.1524) (layer F.Cu) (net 5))
 (segment (start 165.9857 102.619) (end 165.9857 104.569) (width 0.1524) (layer F.Cu) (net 5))
 (segment (start 164.882 104.569) (end 165.9857 104.569) (width 0.1524) (layer F.Cu) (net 5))
 (segment (start 164.882 107.169) (end 165.9857 107.169) (width 0.1524) (layer F.Cu) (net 5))
 (segment (start 164.3302 107.169) (end 164.882 107.169) (width 0.1524) (layer F.Cu) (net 5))
 (segment (start 164.3302 107.169) (end 163.7783 107.169) (width 0.1524) (layer F.Cu) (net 5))
 (segment (start 164.882 107.819) (end 163.7783 107.819) (width 0.1524) (layer F.Cu) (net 5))
 (segment (start 163.7783 107.819) (end 163.7783 107.169) (width 0.1524) (layer F.Cu) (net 5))
 (via (at 170.5908 106.1662) (size 0.6858) (layers F.Cu B.Cu) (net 5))
 (segment (start 144.764 108.839) (end 145.416 108.839) (width 0.1524) (layer F.Cu) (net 15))
 (segment (start 145.416 108.839) (end 146.311 107.944) (width 0.1524) (layer F.Cu) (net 15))
 (segment (start 146.311 107.944) (end 152.357 107.944) (width 0.1524) (layer F.Cu) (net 15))
 (segment (start 152.357 107.944) (end 155.435 104.866) (width 0.1524) (layer F.Cu) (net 15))
 (segment (start 155.435 104.866) (end 161.985 104.866) (width 0.1524) (layer F.Cu) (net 15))
 (segment (start 161.985 104.866) (end 163.778 103.073) (width 0.1524) (layer F.Cu) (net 15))
 (segment (start 163.778 103.073) (end 163.778 102.045) (width 0.1524) (layer F.Cu) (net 15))
 (segment (start 163.778 102.045) (end 163.855 101.969) (width 0.1524) (layer F.Cu) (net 15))
 (segment (start 163.855 101.969) (end 164.882 101.969) (width 0.1524) (layer F.Cu) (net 15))
 (segment (start 158.658 110.894) (end 156.932 110.894) (width 0.1524) (layer F.Cu) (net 13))
 (segment (start 164.882 105.869) (end 163.855 105.869) (width 0.1524) (layer F.Cu) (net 14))
 (segment (start 163.855 105.869) (end 161.584 108.14) (width 0.1524) (layer F.Cu) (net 14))
 (segment (start 161.584 108.14) (end 161.584 110.818) (width 0.1524) (layer F.Cu) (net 14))
 (segment (start 161.584 110.818) (end 161.508 110.894) (width 0.1524) (layer F.Cu) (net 14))
 (segment (start 161.508 110.894) (end 160.756 110.894) (width 0.1524) (layer F.Cu) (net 14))
 (segment (start 157.7659 108.63) (end 157.8299 108.694) (width 0.1524) (layer F.Cu) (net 11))
 (segment (start 157.7659 108.63) (end 158.538 108.63) (width 0.25) (layer F.Cu) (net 11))
 (segment (start 158.538 108.63) (end 158.601 108.567) (width 0.25) (layer F.Cu) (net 11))
 (segment (start 157.728 108.63) (end 157.7659 108.63) (width 0.25) (layer F.Cu) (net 11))
 (segment (start 158.658 108.694) (end 157.8299 108.694) (width 0.1524) (layer F.Cu) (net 11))
 (segment (start 156.918 108.63) (end 157.728 108.63) (width 0.25) (layer F.Cu) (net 11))
 (segment (start 160.756 108.694) (end 160.756 107.942) (width 0.1524) (layer F.Cu) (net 12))
 (segment (start 160.756 107.942) (end 163.479 105.219) (width 0.1524) (layer F.Cu) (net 12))
 (segment (start 163.479 105.219) (end 164.882 105.219) (width 0.1524) (layer F.Cu) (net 12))
 (segment (start 156.906 101.282) (end 158.59 101.282) (width 0.25) (layer F.Cu) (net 16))
 (segment (start 160.9255 101.282) (end 161.163 101.282) (width 0.25) (layer F.Cu) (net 3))
 (segment (start 160.688 101.282) (end 160.9255 101.282) (width 0.25) (layer F.Cu) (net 3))
 (segment (start 160.688 101.282) (end 160.307 101.282) (width 0.1524) (layer F.Cu) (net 3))
 (segment (start 160.9255 101.282) (end 161.163 101.282) (width 0.1524) (layer F.Cu) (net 3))
 (segment (start 160.688 101.282) (end 160.9255 101.282) (width 0.1524) (layer F.Cu) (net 3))
 (segment (start 161.163 101.282) (end 161.62 101.282) (width 0.1524) (layer F.Cu) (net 3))
 (segment (start 161.62 101.282) (end 161.632 101.294) (width 0.1524) (layer F.Cu) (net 3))
 (segment (start 174.782 106.344) (end 174.782 106.644) (width 0.1524) (layer F.Cu) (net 3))
 (segment (start 174.782 105.594) (end 174.782 106.344) (width 0.1524) (layer F.Cu) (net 3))
 (segment (start 160.307 101.282) (end 160.307 100.805) (width 0.2032) (layer F.Cu) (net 3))
 (segment (start 161.26 101.854) (end 160.688 101.282) (width 0.2032) (layer F.Cu) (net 3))
 (segment (start 172.082 107.819) (end 173.907 107.819) (width 0.1524) (layer F.Cu) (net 3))
 (segment (start 173.907 107.819) (end 174.782 106.944) (width 0.1524) (layer F.Cu) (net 3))
 (segment (start 174.782 106.944) (end 174.782 106.644) (width 0.1524) (layer F.Cu) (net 3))
 (segment (start 174.782 106.644) (end 174.782 106.344) (width 0.1524) (layer F.Cu) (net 3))
 (segment (start 181.864 103.251) (end 181.864 104.312) (width 0.1524) (layer B.Cu) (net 3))
 (segment (start 181.864 104.312) (end 180.582 105.594) (width 0.1524) (layer B.Cu) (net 3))
 (segment (start 180.582 105.594) (end 174.782 105.594) (width 0.1524) (layer B.Cu) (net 3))
 (segment (start 161.632 101.294) (end 165.932 105.594) (width 0.1524) (layer B.Cu) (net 3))
 (segment (start 165.932 105.594) (end 174.782 105.594) (width 0.1524) (layer B.Cu) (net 3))
 (via (at 174.782 105.594) (size 0.6858) (layers F.Cu B.Cu) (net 3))
 (via (at 161.632 101.294) (size 0.6858) (layers F.Cu B.Cu) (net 3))
 (segment (start 158.526 103.378) (end 158.527 103.378) (width 0.1524) (layer F.Cu) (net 17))
 (segment (start 156.906 103.378) (end 158.526 103.378) (width 0.25) (layer F.Cu) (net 17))
 (segment (start 174.732 102.944) (end 176.309 104.521) (width 0.1524) (layer F.Cu) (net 4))
 (segment (start 176.309 104.521) (end 179.324 104.521) (width 0.1524) (layer F.Cu) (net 4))
 (segment (start 174.732 102.644) (end 174.732 102.944) (width 0.1524) (layer F.Cu) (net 4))
 (segment (start 160.625 103.378) (end 160.718 103.378) (width 0.2032) (layer F.Cu) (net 4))
 (segment (start 160.244 103.378) (end 160.625 103.378) (width 0.2032) (layer F.Cu) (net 4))
 (segment (start 179.324 105.029) (end 179.324 104.521) (width 0.25) (layer F.Cu) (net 4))
 (segment (start 172.082 103.919) (end 173.757 103.919) (width 0.1524) (layer F.Cu) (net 4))
 (segment (start 173.757 103.919) (end 174.732 102.944) (width 0.1524) (layer F.Cu) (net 4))
 (segment (start 160.625 103.378) (end 163.787 100.215) (width 0.1524) (layer F.Cu) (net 4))
 (segment (start 163.787 100.215) (end 167.351 100.215) (width 0.1524) (layer F.Cu) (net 4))
 (segment (start 167.351 100.215) (end 171.055 103.919) (width 0.1524) (layer F.Cu) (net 4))
 (segment (start 171.055 103.919) (end 172.082 103.919) (width 0.1524) (layer F.Cu) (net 4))
 (segment (start 188.689 104.521) (end 188.021 104.521) (width 0.25) (layer F.Cu) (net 1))
 (segment (start 188.021 104.521) (end 186.624 103.124) (width 0.25) (layer F.Cu) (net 1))
 (segment (start 188.816 104.521) (end 188.689 104.521) (width 0.25) (layer F.Cu) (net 1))
 (segment (start 181.864 100.711) (end 184.211 100.711) (width 0.25) (layer F.Cu) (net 1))
 (segment (start 184.211 100.711) (end 186.624 103.124) (width 0.25) (layer F.Cu) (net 1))
 (segment (start 188.689 105.791) (end 188.153 105.791) (width 0.25) (layer F.Cu) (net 2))
 (segment (start 188.689 105.791) (end 188.153 105.791) (width 0.25) (layer F.Cu) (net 2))
 (segment (start 188.153 105.791) (end 187.391 105.791) (width 0.25) (layer F.Cu) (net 2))
 (segment (start 187.391 105.791) (end 184.724 103.124) (width 0.25) (layer F.Cu) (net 2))
 (segment (start 184.724 103.124) (end 184.404 103.124) (width 0.25) (layer F.Cu) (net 2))
 (segment (start 184.404 103.124) (end 183.261 101.981) (width 0.25) (layer F.Cu) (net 2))
 (segment (start 183.261 101.981) (end 179.324 101.981) (width 0.25) (layer F.Cu) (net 2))
 (segment (start 151.828 106.553) (end 153.317 106.553) (width 0.1524) (layer F.Cu) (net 8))
 (segment (start 153.317 106.553) (end 155.309 104.561) (width 0.1524) (layer F.Cu) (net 8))
 (segment (start 155.309 104.561) (end 161.64 104.561) (width 0.1524) (layer F.Cu) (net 8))
 (segment (start 161.64 104.561) (end 163.474 102.727) (width 0.1524) (layer F.Cu) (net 8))
 (segment (start 163.474 102.727) (end 163.474 101.7) (width 0.1524) (layer F.Cu) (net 8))
 (segment (start 163.474 101.7) (end 163.855 101.319) (width 0.1524) (layer F.Cu) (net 8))
 (segment (start 163.855 101.319) (end 164.882 101.319) (width 0.1524) (layer F.Cu) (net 8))
 (segment (start 150.4099 105.9731) (end 150.4089 105.9731) (width 0.1524) (layer F.Cu) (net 10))
 (segment (start 150.4089 105.9731) (end 149.829 106.553) (width 0.1524) (layer F.Cu) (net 10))
 (segment (start 150.4099 105.9731) (end 151.379 105.004) (width 0.1524) (layer F.Cu) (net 10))
 (segment (start 151.379 105.004) (end 154.435 105.004) (width 0.1524) (layer F.Cu) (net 10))
 (segment (start 154.435 105.004) (end 155.182 104.257) (width 0.1524) (layer F.Cu) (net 10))
 (segment (start 155.182 104.257) (end 161.369 104.257) (width 0.1524) (layer F.Cu) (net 10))
 (segment (start 161.369 104.257) (end 163.169 102.457) (width 0.1524) (layer F.Cu) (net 10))
 (segment (start 163.169 102.457) (end 163.169 101.355) (width 0.1524) (layer F.Cu) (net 10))
 (segment (start 163.169 101.355) (end 163.855 100.669) (width 0.1524) (layer F.Cu) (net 10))
 (segment (start 163.855 100.669) (end 164.882 100.669) (width 0.1524) (layer F.Cu) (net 10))
 (segment (start 149.83 106.553) (end 150.4099 105.9731) (width 0.1524) (layer F.Cu) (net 10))
 (segment (start 149.83 106.6015) (end 149.829 106.6005) (width 0.1524) (layer B.Cu) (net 10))
 (segment (start 149.829 106.6005) (end 149.829 106.553) (width 0.1524) (layer B.Cu) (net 10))
 (segment (start 149.83 106.6015) (end 149.83 106.65) (width 0.25) (layer B.Cu) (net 10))
 (segment (start 149.83 106.553) (end 149.83 106.6015) (width 0.25) (layer B.Cu) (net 10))
 (segment (start 194.089 105.791) (end 195.0927 105.791) (width 0.1524) (layer F.Cu) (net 18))
 (segment (start 194.216 105.156) (end 194.8543 105.156) (width 0.1524) (layer F.Cu) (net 18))
 (segment (start 194.8543 105.156) (end 195.0927 105.3944) (width 0.1524) (layer F.Cu) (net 18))
 (segment (start 195.0927 105.3944) (end 195.0927 105.791) (width 0.1524) (layer F.Cu) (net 18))
 (segment (start 194.216 105.156) (end 194.216 104.521) (width 0.25) (layer F.Cu) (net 18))
 (segment (start 194.216 105.791) (end 194.216 105.156) (width 0.25) (layer F.Cu) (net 18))
 (segment (start 194.089 104.521) (end 194.216 104.521) (width 0.1524) (layer F.Cu) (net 18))
 (segment (start 194.089 104.521) (end 193.614 104.521) (width 0.1524) (layer F.Cu) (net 18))
 (segment (start 193.614 104.521) (end 192.832 103.739) (width 0.1524) (layer F.Cu) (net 18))
 (segment (start 192.832 103.739) (end 192.832 102.094) (width 0.1524) (layer F.Cu) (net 18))
 (segment (start 193.99 110.426) (end 193.99 109.73) (width 0.2032) (layer F.Cu) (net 18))
 (segment (start 193.99 109.73) (end 195.39 108.331) (width 0.2032) (layer F.Cu) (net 18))
 (segment (start 195.39 108.331) (end 195.39 106.108) (width 0.2032) (layer F.Cu) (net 18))
 (segment (start 195.39 106.108) (end 195.072 105.791) (width 0.2032) (layer F.Cu) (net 18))
 (segment (start 195.072 105.791) (end 194.216 105.791) (width 0.2032) (layer F.Cu) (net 18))
 (segment (start 172.107 101.344) (end 172.082 101.319) (width 0.1524) (layer F.Cu) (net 18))
 (segment (start 192.832 102.094) (end 180.66 102.094) (width 0.1524) (layer B.Cu) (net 18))
 (segment (start 180.66 102.094) (end 179.794 102.96) (width 0.1524) (layer B.Cu) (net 18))
 (segment (start 179.794 102.96) (end 178.854 102.96) (width 0.1524) (layer B.Cu) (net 18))
 (segment (start 178.854 102.96) (end 177.188 101.294) (width 0.1524) (layer B.Cu) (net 18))
 (segment (start 177.188 101.294) (end 173.382 101.294) (width 0.1524) (layer B.Cu) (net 18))
 (segment (start 173.382 101.294) (end 172.107 101.294) (width 0.1524) (layer F.Cu) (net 18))
 (segment (start 172.107 101.294) (end 172.082 101.319) (width 0.1524) (layer F.Cu) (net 18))
 (via (at 192.832 102.094) (size 0.6858) (layers F.Cu B.Cu) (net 18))
 (via (at 173.382 101.294) (size 0.6858) (layers F.Cu B.Cu) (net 18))
 (segment (start 172.082 109.119) (end 173.457 109.119) (width 0.2032) (layer F.Cu) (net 19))
 (segment (start 173.457 109.119) (end 173.482 109.144) (width 0.2032) (layer F.Cu) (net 19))
 (segment (start 193.834 102.246) (end 193.982 102.394) (width 0.2032) (layer B.Cu) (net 19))
 (segment (start 193.982 102.394) (end 193.982 103.144) (width 0.2032) (layer F.Cu) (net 19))
 (segment (start 193.982 103.144) (end 194.089 103.251) (width 0.2032) (layer F.Cu) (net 19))
 (segment (start 193.982 102.394) (end 189.606 106.77) (width 0.1524) (layer B.Cu) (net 19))
 (segment (start 189.606 106.77) (end 181.106 106.77) (width 0.1524) (layer B.Cu) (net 19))
 (segment (start 181.106 106.77) (end 179.254 108.622) (width 0.1524) (layer B.Cu) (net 19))
 (segment (start 179.254 108.622) (end 174.004 108.622) (width 0.1524) (layer B.Cu) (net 19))
 (segment (start 174.004 108.622) (end 173.482 109.144) (width 0.1524) (layer B.Cu) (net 19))
 (via (at 173.482 109.144) (size 0.6858) (layers F.Cu B.Cu) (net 19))
 (via (at 193.982 102.394) (size 0.6858) (layers F.Cu B.Cu) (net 19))
 (segment (start 172.082 106.519) (end 171.055 106.519) (width 0.1524) (layer F.Cu) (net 21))
 (segment (start 171.055 106.519) (end 170.978 106.595) (width 0.1524) (layer F.Cu) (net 21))
 (segment (start 170.978 106.595) (end 170.978 109.527) (width 0.1524) (layer F.Cu) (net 21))
 (segment (start 170.978 109.527) (end 172.296 110.844) (width 0.1524) (layer F.Cu) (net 21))
 (segment (start 172.296 110.844) (end 181.782 110.844) (width 0.1524) (layer F.Cu) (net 21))
 (segment (start 181.782 110.844) (end 184.607 108.019) (width 0.1524) (layer F.Cu) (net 21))
 (segment (start 184.607 108.019) (end 192.204 108.019) (width 0.1524) (layer F.Cu) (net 21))
 (segment (start 192.204 108.019) (end 193.162 107.061) (width 0.1524) (layer F.Cu) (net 21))
 (segment (start 193.162 107.061) (end 194.089 107.061) (width 0.1524) (layer F.Cu) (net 21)))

